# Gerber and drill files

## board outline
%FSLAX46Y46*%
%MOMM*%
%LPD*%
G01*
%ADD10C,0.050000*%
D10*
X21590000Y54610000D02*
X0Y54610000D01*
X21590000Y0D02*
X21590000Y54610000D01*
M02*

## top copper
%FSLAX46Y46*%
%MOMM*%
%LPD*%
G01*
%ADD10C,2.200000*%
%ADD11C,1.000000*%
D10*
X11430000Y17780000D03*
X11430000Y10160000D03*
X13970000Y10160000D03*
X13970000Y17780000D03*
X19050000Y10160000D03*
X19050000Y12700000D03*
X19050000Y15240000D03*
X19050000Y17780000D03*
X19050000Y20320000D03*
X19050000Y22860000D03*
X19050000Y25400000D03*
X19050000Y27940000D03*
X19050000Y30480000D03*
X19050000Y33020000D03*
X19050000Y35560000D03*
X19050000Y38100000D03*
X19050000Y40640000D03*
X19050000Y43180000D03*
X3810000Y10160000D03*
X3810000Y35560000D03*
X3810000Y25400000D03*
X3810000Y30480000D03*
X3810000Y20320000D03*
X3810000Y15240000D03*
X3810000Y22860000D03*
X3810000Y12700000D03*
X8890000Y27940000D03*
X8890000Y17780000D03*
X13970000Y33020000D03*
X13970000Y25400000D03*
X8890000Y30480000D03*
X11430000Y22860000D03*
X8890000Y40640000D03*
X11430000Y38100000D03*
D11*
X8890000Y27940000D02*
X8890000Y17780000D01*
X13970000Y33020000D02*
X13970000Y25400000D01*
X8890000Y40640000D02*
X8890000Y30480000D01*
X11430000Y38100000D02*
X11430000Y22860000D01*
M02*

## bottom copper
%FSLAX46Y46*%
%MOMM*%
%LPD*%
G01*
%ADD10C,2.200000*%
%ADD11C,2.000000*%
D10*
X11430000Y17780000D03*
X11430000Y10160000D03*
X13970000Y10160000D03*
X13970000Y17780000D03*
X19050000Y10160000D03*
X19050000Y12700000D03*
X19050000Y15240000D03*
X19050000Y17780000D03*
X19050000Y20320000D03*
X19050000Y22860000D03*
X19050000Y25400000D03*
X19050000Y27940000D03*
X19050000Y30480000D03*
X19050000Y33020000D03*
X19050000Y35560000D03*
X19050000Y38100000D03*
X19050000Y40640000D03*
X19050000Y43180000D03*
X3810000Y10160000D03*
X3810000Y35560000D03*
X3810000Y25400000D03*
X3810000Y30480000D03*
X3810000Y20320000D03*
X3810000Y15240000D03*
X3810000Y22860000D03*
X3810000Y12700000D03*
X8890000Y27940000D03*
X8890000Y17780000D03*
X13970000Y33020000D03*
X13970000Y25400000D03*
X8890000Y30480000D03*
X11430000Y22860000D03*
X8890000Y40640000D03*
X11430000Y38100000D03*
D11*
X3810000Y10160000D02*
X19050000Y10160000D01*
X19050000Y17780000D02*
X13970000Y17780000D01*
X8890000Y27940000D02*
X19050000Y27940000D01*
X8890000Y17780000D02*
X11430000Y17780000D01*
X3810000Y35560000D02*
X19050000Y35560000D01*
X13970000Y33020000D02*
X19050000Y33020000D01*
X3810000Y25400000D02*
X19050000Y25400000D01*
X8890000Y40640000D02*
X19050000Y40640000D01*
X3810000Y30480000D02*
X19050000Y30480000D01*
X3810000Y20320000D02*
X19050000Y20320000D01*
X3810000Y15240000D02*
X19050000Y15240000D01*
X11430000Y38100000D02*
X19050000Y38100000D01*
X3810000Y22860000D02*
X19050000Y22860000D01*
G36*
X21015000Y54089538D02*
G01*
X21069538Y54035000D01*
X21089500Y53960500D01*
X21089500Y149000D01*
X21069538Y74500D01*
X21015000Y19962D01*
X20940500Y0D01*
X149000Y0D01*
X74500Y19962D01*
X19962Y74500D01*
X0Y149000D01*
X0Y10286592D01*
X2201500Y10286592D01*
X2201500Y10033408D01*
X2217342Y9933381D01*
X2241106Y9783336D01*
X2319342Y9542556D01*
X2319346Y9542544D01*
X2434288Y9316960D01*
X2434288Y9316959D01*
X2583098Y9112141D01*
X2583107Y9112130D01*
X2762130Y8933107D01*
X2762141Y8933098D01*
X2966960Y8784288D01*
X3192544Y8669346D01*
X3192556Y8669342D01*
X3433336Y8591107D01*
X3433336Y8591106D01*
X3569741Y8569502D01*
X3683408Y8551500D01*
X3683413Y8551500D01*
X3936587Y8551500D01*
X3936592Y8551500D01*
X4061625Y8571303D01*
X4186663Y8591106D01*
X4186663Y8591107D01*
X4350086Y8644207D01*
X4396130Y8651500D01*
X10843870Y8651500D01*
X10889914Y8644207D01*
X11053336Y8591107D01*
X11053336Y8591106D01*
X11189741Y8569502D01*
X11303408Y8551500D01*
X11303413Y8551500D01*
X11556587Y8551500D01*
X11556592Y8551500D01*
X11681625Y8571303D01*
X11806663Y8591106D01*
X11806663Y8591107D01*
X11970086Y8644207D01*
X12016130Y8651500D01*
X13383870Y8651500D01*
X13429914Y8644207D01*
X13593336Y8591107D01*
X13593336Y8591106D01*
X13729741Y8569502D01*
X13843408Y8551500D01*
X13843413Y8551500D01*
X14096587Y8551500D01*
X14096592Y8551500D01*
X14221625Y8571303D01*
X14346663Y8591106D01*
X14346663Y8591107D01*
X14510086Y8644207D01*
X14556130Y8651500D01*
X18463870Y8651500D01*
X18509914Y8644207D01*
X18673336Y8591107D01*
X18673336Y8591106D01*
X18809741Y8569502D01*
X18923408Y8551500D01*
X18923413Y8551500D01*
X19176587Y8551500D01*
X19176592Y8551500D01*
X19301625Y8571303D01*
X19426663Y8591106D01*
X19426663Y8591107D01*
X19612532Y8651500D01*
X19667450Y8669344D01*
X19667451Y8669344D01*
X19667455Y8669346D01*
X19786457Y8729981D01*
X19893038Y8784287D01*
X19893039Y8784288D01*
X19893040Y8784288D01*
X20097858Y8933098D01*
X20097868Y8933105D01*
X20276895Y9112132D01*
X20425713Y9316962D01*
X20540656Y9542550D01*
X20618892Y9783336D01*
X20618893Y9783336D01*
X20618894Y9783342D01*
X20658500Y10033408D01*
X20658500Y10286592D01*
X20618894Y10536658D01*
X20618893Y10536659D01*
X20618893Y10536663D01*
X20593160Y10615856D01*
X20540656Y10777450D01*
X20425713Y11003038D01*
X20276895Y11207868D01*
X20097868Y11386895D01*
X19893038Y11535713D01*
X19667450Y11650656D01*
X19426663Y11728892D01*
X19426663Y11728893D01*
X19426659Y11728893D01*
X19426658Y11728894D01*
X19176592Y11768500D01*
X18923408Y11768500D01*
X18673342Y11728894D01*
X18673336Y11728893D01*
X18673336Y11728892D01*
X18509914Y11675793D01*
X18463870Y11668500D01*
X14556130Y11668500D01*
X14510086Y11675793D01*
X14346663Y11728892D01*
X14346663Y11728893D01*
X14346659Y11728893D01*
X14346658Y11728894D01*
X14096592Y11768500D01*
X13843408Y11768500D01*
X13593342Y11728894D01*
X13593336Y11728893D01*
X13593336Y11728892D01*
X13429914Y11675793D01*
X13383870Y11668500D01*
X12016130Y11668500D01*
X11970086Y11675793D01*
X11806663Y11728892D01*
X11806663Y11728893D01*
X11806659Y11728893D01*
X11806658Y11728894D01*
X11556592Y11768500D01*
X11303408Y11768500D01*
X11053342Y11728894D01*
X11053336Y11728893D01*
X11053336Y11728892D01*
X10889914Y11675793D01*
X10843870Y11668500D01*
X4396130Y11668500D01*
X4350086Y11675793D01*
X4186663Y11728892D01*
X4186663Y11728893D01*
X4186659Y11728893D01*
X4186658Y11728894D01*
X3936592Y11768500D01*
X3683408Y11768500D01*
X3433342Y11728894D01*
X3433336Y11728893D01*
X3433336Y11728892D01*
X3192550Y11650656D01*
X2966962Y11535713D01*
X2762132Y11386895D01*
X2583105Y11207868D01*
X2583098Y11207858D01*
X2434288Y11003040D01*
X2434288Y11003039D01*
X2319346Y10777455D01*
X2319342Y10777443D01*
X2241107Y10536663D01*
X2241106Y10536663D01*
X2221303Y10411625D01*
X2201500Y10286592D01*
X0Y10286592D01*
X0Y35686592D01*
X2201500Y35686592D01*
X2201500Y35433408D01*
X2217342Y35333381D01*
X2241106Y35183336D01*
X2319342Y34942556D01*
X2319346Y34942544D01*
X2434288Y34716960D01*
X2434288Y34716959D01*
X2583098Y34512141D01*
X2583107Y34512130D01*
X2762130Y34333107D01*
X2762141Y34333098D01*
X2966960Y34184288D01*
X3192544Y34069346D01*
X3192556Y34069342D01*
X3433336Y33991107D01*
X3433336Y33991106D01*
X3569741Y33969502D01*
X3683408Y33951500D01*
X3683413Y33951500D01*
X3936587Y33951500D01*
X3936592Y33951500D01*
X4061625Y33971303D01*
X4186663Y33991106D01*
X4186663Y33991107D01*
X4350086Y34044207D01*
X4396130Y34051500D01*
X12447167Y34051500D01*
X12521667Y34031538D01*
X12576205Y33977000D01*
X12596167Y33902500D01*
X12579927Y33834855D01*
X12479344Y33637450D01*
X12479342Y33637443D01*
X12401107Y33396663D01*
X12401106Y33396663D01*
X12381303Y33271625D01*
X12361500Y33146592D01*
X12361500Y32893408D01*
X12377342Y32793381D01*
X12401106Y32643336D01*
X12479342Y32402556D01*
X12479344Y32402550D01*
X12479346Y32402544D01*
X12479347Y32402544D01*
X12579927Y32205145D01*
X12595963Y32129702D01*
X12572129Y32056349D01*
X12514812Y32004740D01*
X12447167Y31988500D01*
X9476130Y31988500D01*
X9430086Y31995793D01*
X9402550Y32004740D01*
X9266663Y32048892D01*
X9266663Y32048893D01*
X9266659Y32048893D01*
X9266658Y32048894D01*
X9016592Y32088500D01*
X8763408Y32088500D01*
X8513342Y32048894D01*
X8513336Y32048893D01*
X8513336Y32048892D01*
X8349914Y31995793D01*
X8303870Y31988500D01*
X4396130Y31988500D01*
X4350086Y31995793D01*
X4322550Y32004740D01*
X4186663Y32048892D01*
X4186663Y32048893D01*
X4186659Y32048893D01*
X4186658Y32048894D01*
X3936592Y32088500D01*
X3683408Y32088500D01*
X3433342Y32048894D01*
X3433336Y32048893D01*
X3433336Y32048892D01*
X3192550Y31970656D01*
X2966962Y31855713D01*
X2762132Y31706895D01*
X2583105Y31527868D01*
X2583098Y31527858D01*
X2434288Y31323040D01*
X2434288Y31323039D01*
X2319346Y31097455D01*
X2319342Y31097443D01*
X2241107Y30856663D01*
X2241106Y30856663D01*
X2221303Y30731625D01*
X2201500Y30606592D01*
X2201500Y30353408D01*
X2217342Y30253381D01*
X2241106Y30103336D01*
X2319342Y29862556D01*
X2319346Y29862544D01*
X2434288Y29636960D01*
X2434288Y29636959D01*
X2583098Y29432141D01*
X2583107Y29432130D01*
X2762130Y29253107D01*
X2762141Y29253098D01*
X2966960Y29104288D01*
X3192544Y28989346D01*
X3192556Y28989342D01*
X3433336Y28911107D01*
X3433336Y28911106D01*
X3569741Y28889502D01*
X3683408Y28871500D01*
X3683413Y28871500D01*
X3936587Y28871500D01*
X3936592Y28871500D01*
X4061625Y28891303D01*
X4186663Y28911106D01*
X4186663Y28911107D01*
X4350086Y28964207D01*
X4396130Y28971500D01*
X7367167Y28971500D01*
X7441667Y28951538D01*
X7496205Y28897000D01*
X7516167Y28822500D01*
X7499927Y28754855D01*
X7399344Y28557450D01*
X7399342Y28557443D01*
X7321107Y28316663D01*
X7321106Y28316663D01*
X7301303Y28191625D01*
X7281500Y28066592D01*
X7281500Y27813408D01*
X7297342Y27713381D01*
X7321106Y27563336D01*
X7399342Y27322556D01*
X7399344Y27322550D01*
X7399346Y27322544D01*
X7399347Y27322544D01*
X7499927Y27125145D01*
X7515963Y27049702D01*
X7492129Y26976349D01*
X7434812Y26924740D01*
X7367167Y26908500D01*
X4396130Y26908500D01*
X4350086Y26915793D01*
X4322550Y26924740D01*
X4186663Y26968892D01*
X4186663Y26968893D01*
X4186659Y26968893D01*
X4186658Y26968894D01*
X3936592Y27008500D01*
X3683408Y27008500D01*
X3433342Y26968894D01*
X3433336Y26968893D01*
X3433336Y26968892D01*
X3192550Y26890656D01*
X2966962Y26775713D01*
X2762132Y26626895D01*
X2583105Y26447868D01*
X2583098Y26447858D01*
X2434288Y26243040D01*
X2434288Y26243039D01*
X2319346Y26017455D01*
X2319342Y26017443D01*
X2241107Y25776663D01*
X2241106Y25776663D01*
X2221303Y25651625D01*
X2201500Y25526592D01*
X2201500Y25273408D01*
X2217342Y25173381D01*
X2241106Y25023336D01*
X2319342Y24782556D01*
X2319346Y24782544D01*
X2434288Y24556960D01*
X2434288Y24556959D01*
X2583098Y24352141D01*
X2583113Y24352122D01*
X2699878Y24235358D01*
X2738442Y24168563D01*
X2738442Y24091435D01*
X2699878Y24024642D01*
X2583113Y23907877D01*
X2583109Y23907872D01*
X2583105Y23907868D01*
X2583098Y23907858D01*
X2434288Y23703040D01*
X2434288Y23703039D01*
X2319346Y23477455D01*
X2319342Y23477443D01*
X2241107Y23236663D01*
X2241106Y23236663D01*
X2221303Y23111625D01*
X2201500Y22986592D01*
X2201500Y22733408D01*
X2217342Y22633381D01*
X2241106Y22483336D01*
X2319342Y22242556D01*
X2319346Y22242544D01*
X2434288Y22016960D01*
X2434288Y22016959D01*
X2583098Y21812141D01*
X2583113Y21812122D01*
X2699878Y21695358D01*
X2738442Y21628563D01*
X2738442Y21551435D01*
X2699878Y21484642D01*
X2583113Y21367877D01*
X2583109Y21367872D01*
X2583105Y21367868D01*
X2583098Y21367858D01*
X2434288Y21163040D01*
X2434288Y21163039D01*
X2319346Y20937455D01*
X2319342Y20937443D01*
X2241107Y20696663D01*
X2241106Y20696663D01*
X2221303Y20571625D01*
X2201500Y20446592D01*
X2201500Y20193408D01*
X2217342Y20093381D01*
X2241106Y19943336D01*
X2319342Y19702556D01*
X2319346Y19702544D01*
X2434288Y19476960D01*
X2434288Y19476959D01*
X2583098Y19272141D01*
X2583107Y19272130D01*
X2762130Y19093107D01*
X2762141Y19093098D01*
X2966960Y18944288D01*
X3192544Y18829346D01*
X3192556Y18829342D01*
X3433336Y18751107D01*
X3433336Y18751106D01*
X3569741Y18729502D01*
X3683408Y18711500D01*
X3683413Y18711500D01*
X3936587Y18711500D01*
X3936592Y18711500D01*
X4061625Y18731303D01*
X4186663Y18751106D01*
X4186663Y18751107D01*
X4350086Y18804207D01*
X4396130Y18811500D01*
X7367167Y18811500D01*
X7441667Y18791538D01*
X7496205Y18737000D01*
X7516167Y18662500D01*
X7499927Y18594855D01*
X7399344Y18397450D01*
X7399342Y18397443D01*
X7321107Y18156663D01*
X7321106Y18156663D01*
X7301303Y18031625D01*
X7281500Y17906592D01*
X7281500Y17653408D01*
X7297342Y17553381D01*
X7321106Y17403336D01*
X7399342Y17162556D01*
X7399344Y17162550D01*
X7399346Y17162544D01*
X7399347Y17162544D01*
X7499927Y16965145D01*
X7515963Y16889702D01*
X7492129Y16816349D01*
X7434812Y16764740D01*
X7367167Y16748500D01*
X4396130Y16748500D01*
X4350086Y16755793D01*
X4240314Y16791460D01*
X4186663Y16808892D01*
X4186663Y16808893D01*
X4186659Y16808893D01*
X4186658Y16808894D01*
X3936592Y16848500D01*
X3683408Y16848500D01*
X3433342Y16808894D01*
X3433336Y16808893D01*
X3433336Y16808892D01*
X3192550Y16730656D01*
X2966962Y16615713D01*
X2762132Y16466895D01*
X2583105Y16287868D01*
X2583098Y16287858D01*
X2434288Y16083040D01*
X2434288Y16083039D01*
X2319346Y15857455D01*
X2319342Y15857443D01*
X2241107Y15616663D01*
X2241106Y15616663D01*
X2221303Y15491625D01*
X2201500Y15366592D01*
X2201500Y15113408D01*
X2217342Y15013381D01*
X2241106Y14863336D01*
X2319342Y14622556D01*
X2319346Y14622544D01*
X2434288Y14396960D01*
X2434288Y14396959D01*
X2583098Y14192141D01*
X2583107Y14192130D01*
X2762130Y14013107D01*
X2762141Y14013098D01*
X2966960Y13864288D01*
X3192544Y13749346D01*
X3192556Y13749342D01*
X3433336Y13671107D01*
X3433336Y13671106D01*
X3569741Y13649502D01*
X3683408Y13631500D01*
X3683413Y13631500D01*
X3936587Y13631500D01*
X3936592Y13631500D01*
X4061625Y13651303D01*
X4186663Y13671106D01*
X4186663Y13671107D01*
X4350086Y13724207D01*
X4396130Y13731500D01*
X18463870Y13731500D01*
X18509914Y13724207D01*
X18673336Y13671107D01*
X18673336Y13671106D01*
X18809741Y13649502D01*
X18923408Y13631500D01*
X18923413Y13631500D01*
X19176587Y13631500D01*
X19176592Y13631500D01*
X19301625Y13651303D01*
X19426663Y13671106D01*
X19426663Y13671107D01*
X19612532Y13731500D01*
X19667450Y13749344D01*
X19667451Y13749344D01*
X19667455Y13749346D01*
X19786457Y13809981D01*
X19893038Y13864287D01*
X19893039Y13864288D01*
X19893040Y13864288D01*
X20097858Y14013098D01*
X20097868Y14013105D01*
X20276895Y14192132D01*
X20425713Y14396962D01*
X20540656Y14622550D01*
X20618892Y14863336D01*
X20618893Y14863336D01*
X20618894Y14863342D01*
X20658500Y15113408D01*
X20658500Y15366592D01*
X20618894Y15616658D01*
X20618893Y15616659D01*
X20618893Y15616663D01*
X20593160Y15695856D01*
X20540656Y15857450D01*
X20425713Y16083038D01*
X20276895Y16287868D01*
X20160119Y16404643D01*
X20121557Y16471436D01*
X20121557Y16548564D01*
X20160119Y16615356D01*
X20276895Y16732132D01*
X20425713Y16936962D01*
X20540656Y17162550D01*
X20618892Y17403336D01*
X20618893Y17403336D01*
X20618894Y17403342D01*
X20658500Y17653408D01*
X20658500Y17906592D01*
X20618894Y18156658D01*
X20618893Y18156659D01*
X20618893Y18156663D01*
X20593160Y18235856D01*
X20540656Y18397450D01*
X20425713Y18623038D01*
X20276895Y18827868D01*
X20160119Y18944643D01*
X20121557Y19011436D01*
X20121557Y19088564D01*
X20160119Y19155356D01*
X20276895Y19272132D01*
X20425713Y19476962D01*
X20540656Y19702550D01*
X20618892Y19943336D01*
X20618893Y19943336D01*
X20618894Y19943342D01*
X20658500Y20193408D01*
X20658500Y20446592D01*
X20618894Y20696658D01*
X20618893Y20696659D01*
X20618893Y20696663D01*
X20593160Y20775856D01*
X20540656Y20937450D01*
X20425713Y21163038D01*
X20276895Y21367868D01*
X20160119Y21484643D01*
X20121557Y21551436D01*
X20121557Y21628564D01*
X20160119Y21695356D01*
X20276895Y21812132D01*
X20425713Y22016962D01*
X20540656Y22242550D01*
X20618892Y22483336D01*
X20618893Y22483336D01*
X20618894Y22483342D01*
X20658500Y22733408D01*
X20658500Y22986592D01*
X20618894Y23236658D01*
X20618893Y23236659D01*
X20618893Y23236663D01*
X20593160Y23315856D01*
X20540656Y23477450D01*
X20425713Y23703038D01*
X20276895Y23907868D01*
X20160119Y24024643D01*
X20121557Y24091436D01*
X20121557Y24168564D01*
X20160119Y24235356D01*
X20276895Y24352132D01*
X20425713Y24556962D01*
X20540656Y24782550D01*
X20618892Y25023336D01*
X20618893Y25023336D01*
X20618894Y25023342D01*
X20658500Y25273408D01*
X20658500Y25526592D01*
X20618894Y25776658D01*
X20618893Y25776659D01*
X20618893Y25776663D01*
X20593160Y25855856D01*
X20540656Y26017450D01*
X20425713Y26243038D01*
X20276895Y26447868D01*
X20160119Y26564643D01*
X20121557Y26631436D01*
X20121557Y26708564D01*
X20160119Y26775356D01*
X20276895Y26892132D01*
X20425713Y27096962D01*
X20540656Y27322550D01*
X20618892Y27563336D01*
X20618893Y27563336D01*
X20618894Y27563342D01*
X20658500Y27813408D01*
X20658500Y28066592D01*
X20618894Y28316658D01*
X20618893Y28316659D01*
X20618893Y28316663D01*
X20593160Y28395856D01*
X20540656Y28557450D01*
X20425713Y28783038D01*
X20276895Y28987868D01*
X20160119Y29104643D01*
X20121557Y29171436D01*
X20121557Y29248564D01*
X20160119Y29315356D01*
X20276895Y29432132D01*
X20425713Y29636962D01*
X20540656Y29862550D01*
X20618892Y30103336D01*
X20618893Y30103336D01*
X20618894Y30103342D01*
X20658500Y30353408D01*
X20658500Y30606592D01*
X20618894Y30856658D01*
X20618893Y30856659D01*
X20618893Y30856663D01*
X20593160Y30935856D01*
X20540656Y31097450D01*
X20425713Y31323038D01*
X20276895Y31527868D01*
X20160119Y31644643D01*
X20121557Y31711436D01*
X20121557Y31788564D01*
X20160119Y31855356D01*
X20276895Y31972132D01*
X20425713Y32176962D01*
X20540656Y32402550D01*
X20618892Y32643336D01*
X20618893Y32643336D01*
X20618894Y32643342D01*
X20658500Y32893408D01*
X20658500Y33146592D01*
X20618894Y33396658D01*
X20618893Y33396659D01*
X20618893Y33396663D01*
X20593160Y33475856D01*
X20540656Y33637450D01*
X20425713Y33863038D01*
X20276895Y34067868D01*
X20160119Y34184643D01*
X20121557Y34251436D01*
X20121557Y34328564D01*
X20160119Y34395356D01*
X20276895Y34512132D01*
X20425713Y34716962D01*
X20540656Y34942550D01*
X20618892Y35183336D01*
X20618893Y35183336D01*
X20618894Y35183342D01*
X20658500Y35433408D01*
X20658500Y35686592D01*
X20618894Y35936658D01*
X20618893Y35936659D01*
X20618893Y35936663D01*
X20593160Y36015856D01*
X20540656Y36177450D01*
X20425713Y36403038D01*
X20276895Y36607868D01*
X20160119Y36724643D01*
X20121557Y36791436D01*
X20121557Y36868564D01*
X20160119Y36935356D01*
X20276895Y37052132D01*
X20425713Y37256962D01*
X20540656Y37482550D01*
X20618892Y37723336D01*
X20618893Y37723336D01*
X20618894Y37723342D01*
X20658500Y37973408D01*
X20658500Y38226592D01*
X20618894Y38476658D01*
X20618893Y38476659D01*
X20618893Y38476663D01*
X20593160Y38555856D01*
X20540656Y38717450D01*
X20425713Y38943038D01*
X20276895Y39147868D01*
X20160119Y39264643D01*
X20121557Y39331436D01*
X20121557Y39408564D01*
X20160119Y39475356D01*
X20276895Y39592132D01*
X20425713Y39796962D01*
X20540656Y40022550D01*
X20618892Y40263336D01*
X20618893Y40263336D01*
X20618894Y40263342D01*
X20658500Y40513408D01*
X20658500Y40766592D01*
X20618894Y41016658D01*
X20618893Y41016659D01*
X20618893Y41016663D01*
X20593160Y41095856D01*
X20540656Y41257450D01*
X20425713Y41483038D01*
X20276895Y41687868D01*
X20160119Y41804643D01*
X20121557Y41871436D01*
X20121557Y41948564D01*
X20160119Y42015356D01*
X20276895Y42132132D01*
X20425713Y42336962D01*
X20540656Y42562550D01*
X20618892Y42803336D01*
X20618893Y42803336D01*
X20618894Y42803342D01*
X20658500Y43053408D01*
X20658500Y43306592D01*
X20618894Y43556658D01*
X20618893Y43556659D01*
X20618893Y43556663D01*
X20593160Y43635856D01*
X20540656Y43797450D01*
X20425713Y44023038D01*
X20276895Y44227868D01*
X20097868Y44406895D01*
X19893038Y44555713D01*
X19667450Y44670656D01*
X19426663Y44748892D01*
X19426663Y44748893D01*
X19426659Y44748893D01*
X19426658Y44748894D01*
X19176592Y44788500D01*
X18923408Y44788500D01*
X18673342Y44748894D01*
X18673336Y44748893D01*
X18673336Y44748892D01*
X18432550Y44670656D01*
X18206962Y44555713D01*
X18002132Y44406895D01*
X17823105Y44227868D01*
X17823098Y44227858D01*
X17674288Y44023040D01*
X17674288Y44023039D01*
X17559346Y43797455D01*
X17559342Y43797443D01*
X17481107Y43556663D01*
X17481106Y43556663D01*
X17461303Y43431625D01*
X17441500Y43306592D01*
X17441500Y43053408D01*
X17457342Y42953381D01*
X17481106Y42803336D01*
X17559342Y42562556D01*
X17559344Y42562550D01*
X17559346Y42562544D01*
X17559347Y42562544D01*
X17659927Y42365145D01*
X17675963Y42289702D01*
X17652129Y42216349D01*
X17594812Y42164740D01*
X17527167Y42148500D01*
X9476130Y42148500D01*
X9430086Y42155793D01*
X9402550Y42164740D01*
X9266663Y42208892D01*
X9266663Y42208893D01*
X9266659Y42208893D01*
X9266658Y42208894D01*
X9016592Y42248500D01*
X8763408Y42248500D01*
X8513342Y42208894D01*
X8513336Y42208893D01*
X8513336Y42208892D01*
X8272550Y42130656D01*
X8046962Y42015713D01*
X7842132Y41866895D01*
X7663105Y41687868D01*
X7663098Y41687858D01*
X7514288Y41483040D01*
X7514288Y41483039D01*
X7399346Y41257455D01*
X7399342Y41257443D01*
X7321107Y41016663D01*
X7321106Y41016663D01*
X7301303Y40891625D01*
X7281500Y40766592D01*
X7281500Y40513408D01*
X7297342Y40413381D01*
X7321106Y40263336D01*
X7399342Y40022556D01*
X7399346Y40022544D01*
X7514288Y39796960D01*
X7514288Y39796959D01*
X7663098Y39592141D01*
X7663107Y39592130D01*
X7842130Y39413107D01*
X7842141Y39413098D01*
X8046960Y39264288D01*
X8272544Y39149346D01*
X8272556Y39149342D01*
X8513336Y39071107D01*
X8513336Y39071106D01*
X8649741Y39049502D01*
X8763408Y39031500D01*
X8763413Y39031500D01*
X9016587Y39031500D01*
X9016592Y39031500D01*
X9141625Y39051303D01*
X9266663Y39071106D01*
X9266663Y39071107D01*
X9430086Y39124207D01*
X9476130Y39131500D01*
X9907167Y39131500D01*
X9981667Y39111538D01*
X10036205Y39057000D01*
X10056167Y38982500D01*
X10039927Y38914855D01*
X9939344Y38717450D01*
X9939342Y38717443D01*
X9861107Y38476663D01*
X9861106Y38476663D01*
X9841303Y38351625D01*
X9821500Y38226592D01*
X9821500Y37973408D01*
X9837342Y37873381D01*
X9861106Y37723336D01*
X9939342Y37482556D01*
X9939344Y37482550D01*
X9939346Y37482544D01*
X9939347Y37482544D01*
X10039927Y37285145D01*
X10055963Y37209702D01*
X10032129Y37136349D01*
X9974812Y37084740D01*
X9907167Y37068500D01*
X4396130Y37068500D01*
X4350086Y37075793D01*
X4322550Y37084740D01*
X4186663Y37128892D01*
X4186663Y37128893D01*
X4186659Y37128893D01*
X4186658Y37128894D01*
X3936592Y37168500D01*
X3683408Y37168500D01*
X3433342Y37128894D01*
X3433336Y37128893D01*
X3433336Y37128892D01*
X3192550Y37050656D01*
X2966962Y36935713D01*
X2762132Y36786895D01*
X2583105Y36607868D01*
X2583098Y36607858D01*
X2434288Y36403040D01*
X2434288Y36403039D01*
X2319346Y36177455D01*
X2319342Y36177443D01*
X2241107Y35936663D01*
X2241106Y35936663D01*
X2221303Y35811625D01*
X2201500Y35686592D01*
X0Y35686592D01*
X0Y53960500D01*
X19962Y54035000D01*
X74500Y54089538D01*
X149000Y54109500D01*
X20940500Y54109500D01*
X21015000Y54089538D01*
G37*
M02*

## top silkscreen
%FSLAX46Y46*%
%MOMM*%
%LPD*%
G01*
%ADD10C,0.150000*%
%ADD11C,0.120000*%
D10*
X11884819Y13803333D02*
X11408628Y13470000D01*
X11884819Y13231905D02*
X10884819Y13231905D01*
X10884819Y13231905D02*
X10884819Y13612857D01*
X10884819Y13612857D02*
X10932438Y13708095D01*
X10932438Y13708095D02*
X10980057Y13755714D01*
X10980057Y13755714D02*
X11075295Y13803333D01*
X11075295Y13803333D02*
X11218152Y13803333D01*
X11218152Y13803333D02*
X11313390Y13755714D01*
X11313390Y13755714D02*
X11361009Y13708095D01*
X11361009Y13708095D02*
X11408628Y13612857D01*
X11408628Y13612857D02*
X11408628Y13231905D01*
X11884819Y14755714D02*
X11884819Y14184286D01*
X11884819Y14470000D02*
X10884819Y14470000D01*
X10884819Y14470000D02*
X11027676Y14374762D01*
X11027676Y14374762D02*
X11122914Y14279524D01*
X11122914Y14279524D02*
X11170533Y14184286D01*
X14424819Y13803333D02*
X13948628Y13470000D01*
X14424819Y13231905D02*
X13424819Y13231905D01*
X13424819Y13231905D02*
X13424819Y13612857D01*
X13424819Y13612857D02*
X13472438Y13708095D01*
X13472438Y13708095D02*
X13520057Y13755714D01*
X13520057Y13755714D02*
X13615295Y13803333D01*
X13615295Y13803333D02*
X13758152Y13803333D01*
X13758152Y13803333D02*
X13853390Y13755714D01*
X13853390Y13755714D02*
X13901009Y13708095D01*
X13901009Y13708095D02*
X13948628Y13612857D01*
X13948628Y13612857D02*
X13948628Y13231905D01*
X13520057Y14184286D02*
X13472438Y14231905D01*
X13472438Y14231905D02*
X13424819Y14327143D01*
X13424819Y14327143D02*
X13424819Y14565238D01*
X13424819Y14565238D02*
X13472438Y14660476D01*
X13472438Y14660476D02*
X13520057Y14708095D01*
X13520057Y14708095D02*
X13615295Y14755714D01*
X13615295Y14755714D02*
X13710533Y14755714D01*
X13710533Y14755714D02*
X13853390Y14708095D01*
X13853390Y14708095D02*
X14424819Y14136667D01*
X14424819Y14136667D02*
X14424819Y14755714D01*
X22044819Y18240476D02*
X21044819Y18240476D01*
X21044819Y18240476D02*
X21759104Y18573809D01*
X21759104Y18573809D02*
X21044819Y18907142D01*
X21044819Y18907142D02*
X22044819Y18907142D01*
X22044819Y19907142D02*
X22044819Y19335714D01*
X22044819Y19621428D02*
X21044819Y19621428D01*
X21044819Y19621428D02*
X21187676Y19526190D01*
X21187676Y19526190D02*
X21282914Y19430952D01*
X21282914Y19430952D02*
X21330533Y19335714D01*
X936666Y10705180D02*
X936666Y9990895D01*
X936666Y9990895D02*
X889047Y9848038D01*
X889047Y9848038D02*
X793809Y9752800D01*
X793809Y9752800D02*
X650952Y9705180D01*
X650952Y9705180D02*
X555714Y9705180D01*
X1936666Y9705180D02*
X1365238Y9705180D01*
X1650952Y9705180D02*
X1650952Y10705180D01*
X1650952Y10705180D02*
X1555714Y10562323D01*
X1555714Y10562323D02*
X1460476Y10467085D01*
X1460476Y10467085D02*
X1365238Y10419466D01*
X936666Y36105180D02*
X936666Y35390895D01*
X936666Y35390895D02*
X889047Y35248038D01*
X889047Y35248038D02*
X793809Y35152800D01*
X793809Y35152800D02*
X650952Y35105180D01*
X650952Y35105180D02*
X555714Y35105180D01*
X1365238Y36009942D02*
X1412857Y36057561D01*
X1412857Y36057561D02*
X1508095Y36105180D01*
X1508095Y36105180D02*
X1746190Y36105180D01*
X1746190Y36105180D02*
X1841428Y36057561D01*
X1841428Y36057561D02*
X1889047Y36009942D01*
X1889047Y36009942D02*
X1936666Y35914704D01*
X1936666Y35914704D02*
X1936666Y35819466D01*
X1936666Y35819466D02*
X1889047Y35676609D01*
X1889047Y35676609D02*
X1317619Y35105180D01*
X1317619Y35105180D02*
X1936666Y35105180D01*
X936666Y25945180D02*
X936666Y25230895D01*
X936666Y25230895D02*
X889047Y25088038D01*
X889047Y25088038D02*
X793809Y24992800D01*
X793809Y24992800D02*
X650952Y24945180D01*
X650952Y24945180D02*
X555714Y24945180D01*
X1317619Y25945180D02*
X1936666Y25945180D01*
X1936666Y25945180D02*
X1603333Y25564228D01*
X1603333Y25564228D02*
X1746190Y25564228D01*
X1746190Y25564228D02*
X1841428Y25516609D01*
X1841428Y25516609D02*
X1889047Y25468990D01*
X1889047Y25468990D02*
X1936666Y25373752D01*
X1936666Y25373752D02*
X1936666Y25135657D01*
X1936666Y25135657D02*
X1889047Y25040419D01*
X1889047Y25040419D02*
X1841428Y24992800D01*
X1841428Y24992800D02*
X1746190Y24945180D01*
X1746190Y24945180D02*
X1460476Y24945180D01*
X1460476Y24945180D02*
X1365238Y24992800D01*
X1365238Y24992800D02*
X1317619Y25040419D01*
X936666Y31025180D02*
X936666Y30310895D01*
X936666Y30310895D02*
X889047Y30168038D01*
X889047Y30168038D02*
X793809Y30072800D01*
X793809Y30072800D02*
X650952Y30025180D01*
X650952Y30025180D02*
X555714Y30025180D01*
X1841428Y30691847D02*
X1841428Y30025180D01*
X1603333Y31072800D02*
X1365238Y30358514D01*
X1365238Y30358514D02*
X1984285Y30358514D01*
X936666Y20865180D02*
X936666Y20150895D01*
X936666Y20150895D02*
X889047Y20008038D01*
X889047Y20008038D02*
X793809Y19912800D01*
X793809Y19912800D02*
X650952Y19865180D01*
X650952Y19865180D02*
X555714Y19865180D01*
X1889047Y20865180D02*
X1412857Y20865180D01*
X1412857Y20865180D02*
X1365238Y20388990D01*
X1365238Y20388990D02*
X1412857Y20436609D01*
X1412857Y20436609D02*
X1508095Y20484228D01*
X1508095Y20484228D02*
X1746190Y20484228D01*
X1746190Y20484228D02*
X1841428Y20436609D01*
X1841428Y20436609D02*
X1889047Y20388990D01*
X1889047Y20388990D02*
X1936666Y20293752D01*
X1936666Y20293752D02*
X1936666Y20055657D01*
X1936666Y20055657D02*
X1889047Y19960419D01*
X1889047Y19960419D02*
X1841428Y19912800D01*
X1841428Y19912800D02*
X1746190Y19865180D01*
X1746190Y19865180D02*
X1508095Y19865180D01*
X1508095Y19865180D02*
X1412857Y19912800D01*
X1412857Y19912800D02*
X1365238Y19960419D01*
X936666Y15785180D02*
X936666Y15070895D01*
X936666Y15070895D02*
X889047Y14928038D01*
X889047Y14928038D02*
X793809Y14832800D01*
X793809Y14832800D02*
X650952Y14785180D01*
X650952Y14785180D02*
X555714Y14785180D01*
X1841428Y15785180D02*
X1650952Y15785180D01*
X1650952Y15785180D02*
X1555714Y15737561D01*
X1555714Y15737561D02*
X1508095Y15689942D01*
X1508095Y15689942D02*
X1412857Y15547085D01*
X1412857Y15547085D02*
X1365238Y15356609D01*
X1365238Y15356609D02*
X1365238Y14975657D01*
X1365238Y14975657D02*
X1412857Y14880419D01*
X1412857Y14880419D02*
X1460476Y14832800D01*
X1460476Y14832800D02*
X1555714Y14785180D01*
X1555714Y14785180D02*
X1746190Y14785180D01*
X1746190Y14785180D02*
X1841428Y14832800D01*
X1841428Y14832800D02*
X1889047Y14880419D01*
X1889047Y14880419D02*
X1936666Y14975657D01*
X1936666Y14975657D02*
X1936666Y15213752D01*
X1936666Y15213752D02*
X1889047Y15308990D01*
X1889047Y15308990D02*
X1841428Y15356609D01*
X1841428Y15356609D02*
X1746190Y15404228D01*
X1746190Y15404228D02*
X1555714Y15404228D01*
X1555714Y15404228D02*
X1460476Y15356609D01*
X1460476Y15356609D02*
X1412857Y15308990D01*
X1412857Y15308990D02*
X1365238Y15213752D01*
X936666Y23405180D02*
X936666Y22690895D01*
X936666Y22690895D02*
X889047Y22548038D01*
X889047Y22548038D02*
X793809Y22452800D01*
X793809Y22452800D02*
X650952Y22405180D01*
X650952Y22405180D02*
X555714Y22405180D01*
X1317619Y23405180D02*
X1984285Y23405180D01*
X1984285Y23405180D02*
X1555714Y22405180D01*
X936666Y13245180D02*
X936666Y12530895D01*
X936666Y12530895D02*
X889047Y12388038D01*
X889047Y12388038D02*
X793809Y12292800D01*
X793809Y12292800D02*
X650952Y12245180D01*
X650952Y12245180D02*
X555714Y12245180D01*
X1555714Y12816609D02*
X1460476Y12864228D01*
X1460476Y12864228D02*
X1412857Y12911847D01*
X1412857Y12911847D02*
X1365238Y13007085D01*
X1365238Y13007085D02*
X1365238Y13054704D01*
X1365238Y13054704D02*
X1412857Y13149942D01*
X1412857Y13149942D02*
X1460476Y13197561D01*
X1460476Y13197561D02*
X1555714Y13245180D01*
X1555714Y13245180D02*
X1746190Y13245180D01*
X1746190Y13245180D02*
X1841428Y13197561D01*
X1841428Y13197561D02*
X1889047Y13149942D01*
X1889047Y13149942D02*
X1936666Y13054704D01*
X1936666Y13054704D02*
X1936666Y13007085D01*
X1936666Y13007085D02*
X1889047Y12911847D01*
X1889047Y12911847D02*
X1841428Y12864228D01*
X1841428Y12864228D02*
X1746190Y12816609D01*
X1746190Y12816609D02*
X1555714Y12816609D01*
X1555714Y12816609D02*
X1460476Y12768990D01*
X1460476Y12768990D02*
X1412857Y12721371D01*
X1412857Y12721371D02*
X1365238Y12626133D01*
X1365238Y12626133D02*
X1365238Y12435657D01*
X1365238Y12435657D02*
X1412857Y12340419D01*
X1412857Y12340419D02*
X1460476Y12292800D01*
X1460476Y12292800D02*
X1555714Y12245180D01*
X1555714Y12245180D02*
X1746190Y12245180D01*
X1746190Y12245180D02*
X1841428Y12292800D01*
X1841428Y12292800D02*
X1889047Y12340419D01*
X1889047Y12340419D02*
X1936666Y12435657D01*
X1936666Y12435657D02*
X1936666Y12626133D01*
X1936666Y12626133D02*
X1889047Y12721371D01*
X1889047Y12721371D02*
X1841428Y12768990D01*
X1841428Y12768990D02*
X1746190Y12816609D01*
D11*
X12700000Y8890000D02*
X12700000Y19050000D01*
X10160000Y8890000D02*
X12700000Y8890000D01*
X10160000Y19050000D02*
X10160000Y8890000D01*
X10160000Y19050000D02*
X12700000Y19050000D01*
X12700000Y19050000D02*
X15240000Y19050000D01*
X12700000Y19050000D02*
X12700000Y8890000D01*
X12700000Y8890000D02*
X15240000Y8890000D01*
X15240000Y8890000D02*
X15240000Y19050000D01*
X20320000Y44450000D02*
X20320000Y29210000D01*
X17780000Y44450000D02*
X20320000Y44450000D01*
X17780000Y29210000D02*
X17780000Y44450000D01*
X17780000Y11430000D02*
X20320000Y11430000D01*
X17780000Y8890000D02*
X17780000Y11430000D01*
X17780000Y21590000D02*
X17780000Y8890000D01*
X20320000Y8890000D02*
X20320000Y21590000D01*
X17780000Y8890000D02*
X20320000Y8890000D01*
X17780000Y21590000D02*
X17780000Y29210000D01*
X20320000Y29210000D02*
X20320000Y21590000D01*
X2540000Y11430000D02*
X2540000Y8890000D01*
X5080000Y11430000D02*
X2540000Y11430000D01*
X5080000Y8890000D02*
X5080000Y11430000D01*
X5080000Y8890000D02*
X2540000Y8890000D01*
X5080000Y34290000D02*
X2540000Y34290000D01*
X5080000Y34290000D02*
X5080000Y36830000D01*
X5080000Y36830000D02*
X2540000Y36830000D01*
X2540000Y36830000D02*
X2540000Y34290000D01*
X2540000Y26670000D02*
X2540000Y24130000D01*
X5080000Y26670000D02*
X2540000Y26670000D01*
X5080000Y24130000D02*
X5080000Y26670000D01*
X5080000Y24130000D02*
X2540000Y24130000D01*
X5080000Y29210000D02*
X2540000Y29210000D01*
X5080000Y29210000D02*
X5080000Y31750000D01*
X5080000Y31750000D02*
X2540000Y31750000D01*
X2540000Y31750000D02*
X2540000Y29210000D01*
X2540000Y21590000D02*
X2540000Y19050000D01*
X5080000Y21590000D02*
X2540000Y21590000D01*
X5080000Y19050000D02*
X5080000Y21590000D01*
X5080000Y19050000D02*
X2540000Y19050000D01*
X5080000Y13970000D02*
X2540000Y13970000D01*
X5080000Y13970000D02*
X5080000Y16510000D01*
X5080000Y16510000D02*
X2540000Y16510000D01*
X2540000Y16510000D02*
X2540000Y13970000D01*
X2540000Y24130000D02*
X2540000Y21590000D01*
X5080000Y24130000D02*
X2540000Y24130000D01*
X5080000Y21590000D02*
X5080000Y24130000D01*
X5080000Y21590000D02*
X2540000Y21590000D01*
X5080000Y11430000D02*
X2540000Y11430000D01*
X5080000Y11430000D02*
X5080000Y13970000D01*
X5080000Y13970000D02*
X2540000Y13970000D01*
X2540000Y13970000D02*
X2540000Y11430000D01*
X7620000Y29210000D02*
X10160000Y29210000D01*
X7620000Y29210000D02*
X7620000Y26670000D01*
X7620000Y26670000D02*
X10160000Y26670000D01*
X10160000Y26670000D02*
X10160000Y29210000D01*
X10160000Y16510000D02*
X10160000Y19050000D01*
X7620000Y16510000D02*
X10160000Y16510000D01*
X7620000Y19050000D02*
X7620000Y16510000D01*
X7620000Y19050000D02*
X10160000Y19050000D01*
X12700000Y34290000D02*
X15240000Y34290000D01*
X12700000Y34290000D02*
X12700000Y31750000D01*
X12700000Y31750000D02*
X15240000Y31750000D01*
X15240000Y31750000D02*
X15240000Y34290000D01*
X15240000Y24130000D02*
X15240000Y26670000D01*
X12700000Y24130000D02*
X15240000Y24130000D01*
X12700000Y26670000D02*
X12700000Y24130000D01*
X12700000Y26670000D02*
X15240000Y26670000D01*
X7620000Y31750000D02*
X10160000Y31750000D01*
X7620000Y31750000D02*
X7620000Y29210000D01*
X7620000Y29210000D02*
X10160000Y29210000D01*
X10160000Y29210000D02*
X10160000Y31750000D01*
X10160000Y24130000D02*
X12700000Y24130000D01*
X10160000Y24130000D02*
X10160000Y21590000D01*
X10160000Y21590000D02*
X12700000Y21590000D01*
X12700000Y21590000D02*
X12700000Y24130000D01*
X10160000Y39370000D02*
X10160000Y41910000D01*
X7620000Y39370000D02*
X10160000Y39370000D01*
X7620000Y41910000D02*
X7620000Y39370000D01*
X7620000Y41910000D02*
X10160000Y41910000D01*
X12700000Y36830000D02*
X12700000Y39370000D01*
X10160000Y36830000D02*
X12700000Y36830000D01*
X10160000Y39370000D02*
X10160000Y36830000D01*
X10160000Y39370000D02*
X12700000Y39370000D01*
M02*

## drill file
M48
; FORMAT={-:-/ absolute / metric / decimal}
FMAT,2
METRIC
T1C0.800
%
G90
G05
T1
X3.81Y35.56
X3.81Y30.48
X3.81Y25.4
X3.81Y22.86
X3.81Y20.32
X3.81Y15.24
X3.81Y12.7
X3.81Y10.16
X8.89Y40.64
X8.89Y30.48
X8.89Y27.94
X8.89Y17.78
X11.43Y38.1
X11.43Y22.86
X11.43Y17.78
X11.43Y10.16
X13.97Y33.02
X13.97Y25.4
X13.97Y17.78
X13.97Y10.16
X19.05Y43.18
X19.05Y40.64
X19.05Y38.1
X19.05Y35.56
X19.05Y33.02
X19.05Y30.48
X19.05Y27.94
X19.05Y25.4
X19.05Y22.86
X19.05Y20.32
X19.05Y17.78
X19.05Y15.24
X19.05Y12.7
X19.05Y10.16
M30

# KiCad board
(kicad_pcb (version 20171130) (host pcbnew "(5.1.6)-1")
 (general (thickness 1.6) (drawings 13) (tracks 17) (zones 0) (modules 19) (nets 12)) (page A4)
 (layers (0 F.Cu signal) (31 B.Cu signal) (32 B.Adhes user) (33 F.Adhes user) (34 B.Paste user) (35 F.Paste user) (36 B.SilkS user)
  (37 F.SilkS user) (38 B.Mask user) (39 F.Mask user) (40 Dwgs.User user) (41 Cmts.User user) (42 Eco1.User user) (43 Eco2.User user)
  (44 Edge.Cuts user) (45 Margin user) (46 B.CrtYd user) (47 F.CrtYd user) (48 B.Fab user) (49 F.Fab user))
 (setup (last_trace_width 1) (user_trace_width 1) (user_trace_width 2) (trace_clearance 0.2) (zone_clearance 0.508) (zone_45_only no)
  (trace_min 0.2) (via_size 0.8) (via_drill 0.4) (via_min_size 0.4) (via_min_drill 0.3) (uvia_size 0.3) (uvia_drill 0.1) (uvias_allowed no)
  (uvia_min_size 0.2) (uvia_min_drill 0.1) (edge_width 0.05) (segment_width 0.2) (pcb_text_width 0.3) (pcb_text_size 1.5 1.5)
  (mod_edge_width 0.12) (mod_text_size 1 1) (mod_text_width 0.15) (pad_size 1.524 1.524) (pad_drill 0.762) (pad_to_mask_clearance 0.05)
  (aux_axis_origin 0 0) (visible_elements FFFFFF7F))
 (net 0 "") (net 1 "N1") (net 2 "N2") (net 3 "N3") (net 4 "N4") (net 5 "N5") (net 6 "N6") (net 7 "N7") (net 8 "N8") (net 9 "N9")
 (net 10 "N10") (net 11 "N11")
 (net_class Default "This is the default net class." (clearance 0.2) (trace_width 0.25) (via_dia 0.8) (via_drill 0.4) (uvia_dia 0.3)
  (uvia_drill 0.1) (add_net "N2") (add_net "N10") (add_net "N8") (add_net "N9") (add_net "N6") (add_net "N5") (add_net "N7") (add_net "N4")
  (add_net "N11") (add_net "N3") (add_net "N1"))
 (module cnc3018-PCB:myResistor (layer F.Cu) (at 11.43 -10.16 90)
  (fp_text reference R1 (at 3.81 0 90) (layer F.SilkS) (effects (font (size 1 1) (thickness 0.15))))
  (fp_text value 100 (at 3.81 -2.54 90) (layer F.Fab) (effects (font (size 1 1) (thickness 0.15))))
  (fp_line (start -1.27 1.27) (end 8.89 1.27) (layer F.SilkS) (width 0.12))
  (fp_line (start -1.27 -1.27) (end -1.27 1.27) (layer F.SilkS) (width 0.12))
  (fp_line (start 8.89 -1.27) (end -1.27 -1.27) (layer F.SilkS) (width 0.12))
  (fp_line (start 8.89 -1.27) (end 8.89 1.27) (layer F.SilkS) (width 0.12))
  (pad 2 thru_hole circle (at 7.62 0 90) (size 2.2 2.2) (drill 0.8) (layers *.Cu *.Mask) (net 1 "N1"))
  (pad 1 thru_hole circle (at 0 0 90) (size 2.2 2.2) (drill 0.8) (layers *.Cu *.Mask) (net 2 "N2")))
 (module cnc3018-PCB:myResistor (layer F.Cu) (at 13.97 -10.16 90)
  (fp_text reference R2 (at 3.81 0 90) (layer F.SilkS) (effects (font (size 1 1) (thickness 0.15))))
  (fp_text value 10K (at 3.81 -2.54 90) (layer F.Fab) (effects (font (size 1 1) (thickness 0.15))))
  (fp_line (start 8.89 -1.27) (end 8.89 1.27) (layer F.SilkS) (width 0.12))
  (fp_line (start 8.89 -1.27) (end -1.27 -1.27) (layer F.SilkS) (width 0.12))
  (fp_line (start -1.27 -1.27) (end -1.27 1.27) (layer F.SilkS) (width 0.12))
  (fp_line (start -1.27 1.27) (end 8.89 1.27) (layer F.SilkS) (width 0.12))
  (pad 1 thru_hole circle (at 0 0 90) (size 2.2 2.2) (drill 0.8) (layers *.Cu *.Mask) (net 2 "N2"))
  (pad 2 thru_hole circle (at 7.62 0 90) (size 2.2 2.2) (drill 0.8) (layers *.Cu *.Mask) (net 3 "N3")))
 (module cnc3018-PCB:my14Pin (layer F.Cu) (at 19.05 -17.78 90)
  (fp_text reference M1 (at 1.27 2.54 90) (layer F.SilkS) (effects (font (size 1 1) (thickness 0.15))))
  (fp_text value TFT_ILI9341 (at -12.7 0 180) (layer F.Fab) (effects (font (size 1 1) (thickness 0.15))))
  (fp_line (start 26.67 1.27) (end 11.43 1.27) (layer F.SilkS) (width 0.12))
  (fp_line (start 26.67 -1.27) (end 26.67 1.27) (layer F.SilkS) (width 0.12))
  (fp_line (start 11.43 -1.27) (end 26.67 -1.27) (layer F.SilkS) (width 0.12))
  (fp_line (start -6.35 -1.27) (end -6.35 1.27) (layer F.SilkS) (width 0.12))
  (fp_line (start -8.89 -1.27) (end -6.35 -1.27) (layer F.SilkS) (width 0.12))
  (fp_line (start 3.81 -1.27) (end -8.89 -1.27) (layer F.SilkS) (width 0.12))
  (fp_line (start -8.89 1.27) (end 3.81 1.27) (layer F.SilkS) (width 0.12))
  (fp_line (start -8.89 -1.27) (end -8.89 1.27) (layer F.SilkS) (width 0.12))
  (fp_line (start 3.81 -1.27) (end 11.43 -1.27) (layer F.SilkS) (width 0.12))
  (fp_line (start 11.43 1.27) (end 3.81 1.27) (layer F.SilkS) (width 0.12))
  (pad 1 thru_hole circle (at -7.62 0 90) (size 2.2 2.2) (drill 0.8) (layers *.Cu *.Mask) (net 2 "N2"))
  (pad 2 thru_hole circle (at -5.08 0 90) (size 2.2 2.2) (drill 0.8) (layers *.Cu *.Mask) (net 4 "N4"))
  (pad 3 thru_hole circle (at -2.54 0 90) (size 2.2 2.2) (drill 0.8) (layers *.Cu *.Mask) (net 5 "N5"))
  (pad 4 thru_hole circle (at 0 0 90) (size 2.2 2.2) (drill 0.8) (layers *.Cu *.Mask) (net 3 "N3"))
  (pad 5 thru_hole circle (at 2.54 0 90) (size 2.2 2.2) (drill 0.8) (layers *.Cu *.Mask) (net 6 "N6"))
  (pad 6 thru_hole circle (at 5.08 0 90) (size 2.2 2.2) (drill 0.8) (layers *.Cu *.Mask) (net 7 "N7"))
  (pad 7 thru_hole circle (at 7.62 0 90) (size 2.2 2.2) (drill 0.8) (layers *.Cu *.Mask) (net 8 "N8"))
  (pad 8 thru_hole circle (at 10.16 0 90) (size 2.2 2.2) (drill 0.8) (layers *.Cu *.Mask) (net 1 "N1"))
  (pad 9 thru_hole circle (at 12.7 0 90) (size 2.2 2.2) (drill 0.8) (layers *.Cu *.Mask) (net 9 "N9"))
  (pad 10 thru_hole circle (at 15.24 0 90) (size 2.2 2.2) (drill 0.8) (layers *.Cu *.Mask) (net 8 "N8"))
  (pad 11 thru_hole circle (at 17.78 0 90) (size 2.2 2.2) (drill 0.8) (layers *.Cu *.Mask) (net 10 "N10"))
  (pad 12 thru_hole circle (at 20.32 0 90) (size 2.2 2.2) (drill 0.8) (layers *.Cu *.Mask) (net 7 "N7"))
  (pad 13 thru_hole circle (at 22.86 0 90) (size 2.2 2.2) (drill 0.8) (layers *.Cu *.Mask) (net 9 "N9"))
  (pad 14 thru_hole circle (at 25.4 0 90) (size 2.2 2.2) (drill 0.8) (layers *.Cu *.Mask) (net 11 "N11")))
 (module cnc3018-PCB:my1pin (layer F.Cu) (at 3.81 -10.16 180)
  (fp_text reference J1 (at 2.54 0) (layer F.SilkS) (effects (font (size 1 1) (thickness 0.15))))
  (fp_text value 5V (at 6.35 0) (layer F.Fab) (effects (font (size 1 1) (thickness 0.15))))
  (fp_line (start 1.27 1.27) (end 1.27 -1.27) (layer F.SilkS) (width 0.12))
  (fp_line (start -1.27 1.27) (end 1.27 1.27) (layer F.SilkS) (width 0.12))
  (fp_line (start -1.27 -1.27) (end -1.27 1.27) (layer F.SilkS) (width 0.12))
  (fp_line (start -1.27 -1.27) (end 1.27 -1.27) (layer F.SilkS) (width 0.12))
  (pad 1 thru_hole circle (at 0 0 180) (size 2.2 2.2) (drill 0.8) (layers *.Cu *.Mask) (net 2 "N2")))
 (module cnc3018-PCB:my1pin (layer F.Cu) (at 3.81 -35.56 180)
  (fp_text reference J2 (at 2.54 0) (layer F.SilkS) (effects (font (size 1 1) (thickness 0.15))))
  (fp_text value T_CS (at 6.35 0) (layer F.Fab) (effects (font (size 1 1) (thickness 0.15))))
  (fp_line (start -1.27 -1.27) (end 1.27 -1.27) (layer F.SilkS) (width 0.12))
  (fp_line (start -1.27 -1.27) (end -1.27 1.27) (layer F.SilkS) (width 0.12))
  (fp_line (start -1.27 1.27) (end 1.27 1.27) (layer F.SilkS) (width 0.12))
  (fp_line (start 1.27 1.27) (end 1.27 -1.27) (layer F.SilkS) (width 0.12))
  (pad 1 thru_hole circle (at 0 0 180) (size 2.2 2.2) (drill 0.8) (layers *.Cu *.Mask) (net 10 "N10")))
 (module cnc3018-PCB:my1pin (layer F.Cu) (at 3.81 -25.4 180)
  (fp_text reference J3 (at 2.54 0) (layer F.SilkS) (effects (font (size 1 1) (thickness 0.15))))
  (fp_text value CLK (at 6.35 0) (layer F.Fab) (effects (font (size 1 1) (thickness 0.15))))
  (fp_line (start 1.27 1.27) (end 1.27 -1.27) (layer F.SilkS) (width 0.12))
  (fp_line (start -1.27 1.27) (end 1.27 1.27) (layer F.SilkS) (width 0.12))
  (fp_line (start -1.27 -1.27) (end -1.27 1.27) (layer F.SilkS) (width 0.12))
  (fp_line (start -1.27 -1.27) (end 1.27 -1.27) (layer F.SilkS) (width 0.12))
  (pad 1 thru_hole circle (at 0 0 180) (size 2.2 2.2) (drill 0.8) (layers *.Cu *.Mask) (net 8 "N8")))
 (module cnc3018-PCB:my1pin (layer F.Cu) (at 3.81 -30.48 180)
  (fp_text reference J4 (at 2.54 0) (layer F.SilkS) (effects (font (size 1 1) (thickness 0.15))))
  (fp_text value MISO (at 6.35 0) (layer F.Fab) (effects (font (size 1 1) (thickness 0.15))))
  (fp_line (start -1.27 -1.27) (end 1.27 -1.27) (layer F.SilkS) (width 0.12))
  (fp_line (start -1.27 -1.27) (end -1.27 1.27) (layer F.SilkS) (width 0.12))
  (fp_line (start -1.27 1.27) (end 1.27 1.27) (layer F.SilkS) (width 0.12))
  (fp_line (start 1.27 1.27) (end 1.27 -1.27) (layer F.SilkS) (width 0.12))
  (pad 1 thru_hole circle (at 0 0 180) (size 2.2 2.2) (drill 0.8) (layers *.Cu *.Mask) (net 9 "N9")))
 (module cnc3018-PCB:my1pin (layer F.Cu) (at 3.81 -20.32 180)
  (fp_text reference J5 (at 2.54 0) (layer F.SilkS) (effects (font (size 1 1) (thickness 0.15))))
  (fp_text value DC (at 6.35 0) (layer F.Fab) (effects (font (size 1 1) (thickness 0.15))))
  (fp_line (start 1.27 1.27) (end 1.27 -1.27) (layer F.SilkS) (width 0.12))
  (fp_line (start -1.27 1.27) (end 1.27 1.27) (layer F.SilkS) (width 0.12))
  (fp_line (start -1.27 -1.27) (end -1.27 1.27) (layer F.SilkS) (width 0.12))
  (fp_line (start -1.27 -1.27) (end 1.27 -1.27) (layer F.SilkS) (width 0.12))
  (pad 1 thru_hole circle (at 0 0 180) (size 2.2 2.2) (drill 0.8) (layers *.Cu *.Mask) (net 6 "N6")))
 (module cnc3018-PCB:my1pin (layer F.Cu) (at 3.81 -15.24 180)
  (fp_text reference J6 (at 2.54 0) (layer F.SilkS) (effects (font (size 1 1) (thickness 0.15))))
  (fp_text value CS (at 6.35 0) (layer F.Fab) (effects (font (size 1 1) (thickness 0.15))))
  (fp_line (start -1.27 -1.27) (end 1.27 -1.27) (layer F.SilkS) (width 0.12))
  (fp_line (start -1.27 -1.27) (end -1.27 1.27) (layer F.SilkS) (width 0.12))
  (fp_line (start -1.27 1.27) (end 1.27 1.27) (layer F.SilkS) (width 0.12))
  (fp_line (start 1.27 1.27) (end 1.27 -1.27) (layer F.SilkS) (width 0.12))
  (pad 1 thru_hole circle (at 0 0 180) (size 2.2 2.2) (drill 0.8) (layers *.Cu *.Mask) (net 5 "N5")))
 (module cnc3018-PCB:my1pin (layer F.Cu) (at 3.81 -22.86 180)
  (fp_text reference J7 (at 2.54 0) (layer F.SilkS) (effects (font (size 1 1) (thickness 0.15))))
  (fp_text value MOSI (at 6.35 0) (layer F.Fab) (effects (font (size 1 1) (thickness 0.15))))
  (fp_line (start 1.27 1.27) (end 1.27 -1.27) (layer F.SilkS) (width 0.12))
  (fp_line (start -1.27 1.27) (end 1.27 1.27) (layer F.SilkS) (width 0.12))
  (fp_line (start -1.27 -1.27) (end -1.27 1.27) (layer F.SilkS) (width 0.12))
  (fp_line (start -1.27 -1.27) (end 1.27 -1.27) (layer F.SilkS) (width 0.12))
  (pad 1 thru_hole circle (at 0 0 180) (size 2.2 2.2) (drill 0.8) (layers *.Cu *.Mask) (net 7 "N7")))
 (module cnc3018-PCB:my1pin (layer F.Cu) (at 3.81 -12.7 180)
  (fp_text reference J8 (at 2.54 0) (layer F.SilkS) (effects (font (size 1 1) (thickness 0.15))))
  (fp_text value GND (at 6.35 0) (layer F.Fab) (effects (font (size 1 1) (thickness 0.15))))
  (fp_line (start -1.27 -1.27) (end 1.27 -1.27) (layer F.SilkS) (width 0.12))
  (fp_line (start -1.27 -1.27) (end -1.27 1.27) (layer F.SilkS) (width 0.12))
  (fp_line (start -1.27 1.27) (end 1.27 1.27) (layer F.SilkS) (width 0.12))
  (fp_line (start 1.27 1.27) (end 1.27 -1.27) (layer F.SilkS) (width 0.12))
  (pad 1 thru_hole circle (at 0 0 180) (size 2.2 2.2) (drill 0.8) (layers *.Cu *.Mask) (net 4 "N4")))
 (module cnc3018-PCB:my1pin (layer F.Cu) (at 8.89 -27.94)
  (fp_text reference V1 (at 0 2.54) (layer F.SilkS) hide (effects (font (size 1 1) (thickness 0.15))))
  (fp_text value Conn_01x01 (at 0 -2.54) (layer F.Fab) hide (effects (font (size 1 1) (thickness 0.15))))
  (fp_line (start -1.27 -1.27) (end 1.27 -1.27) (layer F.SilkS) (width 0.12))
  (fp_line (start -1.27 -1.27) (end -1.27 1.27) (layer F.SilkS) (width 0.12))
  (fp_line (start -1.27 1.27) (end 1.27 1.27) (layer F.SilkS) (width 0.12))
  (fp_line (start 1.27 1.27) (end 1.27 -1.27) (layer F.SilkS) (width 0.12))
  (pad 1 thru_hole circle (at 0 0) (size 2.2 2.2) (drill 0.8) (layers *.Cu *.Mask) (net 1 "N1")))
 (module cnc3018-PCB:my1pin (layer F.Cu) (at 8.89 -17.78)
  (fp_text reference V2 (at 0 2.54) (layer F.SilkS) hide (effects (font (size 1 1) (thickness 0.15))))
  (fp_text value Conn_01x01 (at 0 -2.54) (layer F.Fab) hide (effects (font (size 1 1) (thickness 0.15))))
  (fp_line (start 1.27 1.27) (end 1.27 -1.27) (layer F.SilkS) (width 0.12))
  (fp_line (start -1.27 1.27) (end 1.27 1.27) (layer F.SilkS) (width 0.12))
  (fp_line (start -1.27 -1.27) (end -1.27 1.27) (layer F.SilkS) (width 0.12))
  (fp_line (start -1.27 -1.27) (end 1.27 -1.27) (layer F.SilkS) (width 0.12))
  (pad 1 thru_hole circle (at 0 0) (size 2.2 2.2) (drill 0.8) (layers *.Cu *.Mask) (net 1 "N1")))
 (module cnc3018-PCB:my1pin (layer F.Cu) (at 13.97 -33.02)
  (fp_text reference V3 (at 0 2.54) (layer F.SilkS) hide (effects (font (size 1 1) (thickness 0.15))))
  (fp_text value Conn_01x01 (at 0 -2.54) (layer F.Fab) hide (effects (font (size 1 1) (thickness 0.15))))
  (fp_line (start -1.27 -1.27) (end 1.27 -1.27) (layer F.SilkS) (width 0.12))
  (fp_line (start -1.27 -1.27) (end -1.27 1.27) (layer F.SilkS) (width 0.12))
  (fp_line (start -1.27 1.27) (end 1.27 1.27) (layer F.SilkS) (width 0.12))
  (fp_line (start 1.27 1.27) (end 1.27 -1.27) (layer F.SilkS) (width 0.12))
  (pad 1 thru_hole circle (at 0 0) (size 2.2 2.2) (drill 0.8) (layers *.Cu *.Mask) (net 8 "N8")))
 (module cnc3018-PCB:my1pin (layer F.Cu) (at 13.97 -25.4)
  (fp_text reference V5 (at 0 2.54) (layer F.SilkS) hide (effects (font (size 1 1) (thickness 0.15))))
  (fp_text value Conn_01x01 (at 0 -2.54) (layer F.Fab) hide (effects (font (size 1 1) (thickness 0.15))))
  (fp_line (start 1.27 1.27) (end 1.27 -1.27) (layer F.SilkS) (width 0.12))
  (fp_line (start -1.27 1.27) (end 1.27 1.27) (layer F.SilkS) (width 0.12))
  (fp_line (start -1.27 -1.27) (end -1.27 1.27) (layer F.SilkS) (width 0.12))
  (fp_line (start -1.27 -1.27) (end 1.27 -1.27) (layer F.SilkS) (width 0.12))
  (pad 1 thru_hole circle (at 0 0) (size 2.2 2.2) (drill 0.8) (layers *.Cu *.Mask) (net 8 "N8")))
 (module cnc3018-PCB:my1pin (layer F.Cu) (at 8.89 -30.48)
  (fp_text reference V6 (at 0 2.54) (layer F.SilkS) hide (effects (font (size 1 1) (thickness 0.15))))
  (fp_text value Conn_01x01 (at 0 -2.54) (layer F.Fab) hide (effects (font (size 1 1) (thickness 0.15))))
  (fp_line (start -1.27 -1.27) (end 1.27 -1.27) (layer F.SilkS) (width 0.12))
  (fp_line (start -1.27 -1.27) (end -1.27 1.27) (layer F.SilkS) (width 0.12))
  (fp_line (start -1.27 1.27) (end 1.27 1.27) (layer F.SilkS) (width 0.12))
  (fp_line (start 1.27 1.27) (end 1.27 -1.27) (layer F.SilkS) (width 0.12))
  (pad 1 thru_hole circle (at 0 0) (size 2.2 2.2) (drill 0.8) (layers *.Cu *.Mask) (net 9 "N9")))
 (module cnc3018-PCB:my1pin (layer F.Cu) (at 11.43 -22.86)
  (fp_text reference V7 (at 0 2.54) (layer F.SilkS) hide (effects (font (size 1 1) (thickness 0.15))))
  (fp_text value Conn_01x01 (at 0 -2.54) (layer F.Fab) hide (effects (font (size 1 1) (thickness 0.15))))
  (fp_line (start -1.27 -1.27) (end 1.27 -1.27) (layer F.SilkS) (width 0.12))
  (fp_line (start -1.27 -1.27) (end -1.27 1.27) (layer F.SilkS) (width 0.12))
  (fp_line (start -1.27 1.27) (end 1.27 1.27) (layer F.SilkS) (width 0.12))
  (fp_line (start 1.27 1.27) (end 1.27 -1.27) (layer F.SilkS) (width 0.12))
  (pad 1 thru_hole circle (at 0 0) (size 2.2 2.2) (drill 0.8) (layers *.Cu *.Mask) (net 7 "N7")))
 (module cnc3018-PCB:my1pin (layer F.Cu) (at 8.89 -40.64)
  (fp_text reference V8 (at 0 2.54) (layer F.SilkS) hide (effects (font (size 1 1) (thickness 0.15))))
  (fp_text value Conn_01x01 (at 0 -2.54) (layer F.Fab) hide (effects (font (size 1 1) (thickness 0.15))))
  (fp_line (start 1.27 1.27) (end 1.27 -1.27) (layer F.SilkS) (width 0.12))
  (fp_line (start -1.27 1.27) (end 1.27 1.27) (layer F.SilkS) (width 0.12))
  (fp_line (start -1.27 -1.27) (end -1.27 1.27) (layer F.SilkS) (width 0.12))
  (fp_line (start -1.27 -1.27) (end 1.27 -1.27) (layer F.SilkS) (width 0.12))
  (pad 1 thru_hole circle (at 0 0) (size 2.2 2.2) (drill 0.8) (layers *.Cu *.Mask) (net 9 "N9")))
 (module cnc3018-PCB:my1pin (layer F.Cu) (at 11.43 -38.1)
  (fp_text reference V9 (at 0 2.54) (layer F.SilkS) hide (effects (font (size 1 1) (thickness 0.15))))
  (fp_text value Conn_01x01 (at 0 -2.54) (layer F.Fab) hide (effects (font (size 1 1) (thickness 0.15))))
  (fp_line (start 1.27 1.27) (end 1.27 -1.27) (layer F.SilkS) (width 0.12))
  (fp_line (start -1.27 1.27) (end 1.27 1.27) (layer F.SilkS) (width 0.12))
  (fp_line (start -1.27 -1.27) (end -1.27 1.27) (layer F.SilkS) (width 0.12))
  (fp_line (start -1.27 -1.27) (end 1.27 -1.27) (layer F.SilkS) (width 0.12))
  (pad 1 thru_hole circle (at 0 0) (size 2.2 2.2) (drill 0.8) (layers *.Cu *.Mask) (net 7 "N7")))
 (gr_line (start 21.59 -54.61) (end 0 -54.61) (layer Edge.Cuts) (width 0.05))
 (gr_line (start 21.59 0) (end 21.59 -54.61) (layer Edge.Cuts) (width 0.05))
 (segment (start 3.81 -10.16) (end 19.05 -10.16) (width 2) (layer B.Cu) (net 2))
 (segment (start 19.05 -17.78) (end 13.97 -17.78) (width 2) (layer B.Cu) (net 3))
 (segment (start 8.89 -27.94) (end 19.05 -27.94) (width 2) (layer B.Cu) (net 1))
 (segment (start 8.89 -17.78) (end 11.43 -17.78) (width 2) (layer B.Cu) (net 1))
 (segment (start 8.89 -27.94) (end 8.89 -17.78) (width 1) (layer F.Cu) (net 1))
 (segment (start 3.81 -35.56) (end 19.05 -35.56) (width 2) (layer B.Cu) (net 10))
 (segment (start 13.97 -33.02) (end 19.05 -33.02) (width 2) (layer B.Cu) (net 8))
 (segment (start 3.81 -25.4) (end 19.05 -25.4) (width 2) (layer B.Cu) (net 8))
 (segment (start 13.97 -33.02) (end 13.97 -25.4) (width 1) (layer F.Cu) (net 8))
 (segment (start 8.89 -40.64) (end 19.05 -40.64) (width 2) (layer B.Cu) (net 9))
 (segment (start 3.81 -30.48) (end 19.05 -30.48) (width 2) (layer B.Cu) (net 9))
 (segment (start 8.89 -40.64) (end 8.89 -30.48) (width 1) (layer F.Cu) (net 9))
 (segment (start 3.81 -20.32) (end 19.05 -20.32) (width 2) (layer B.Cu) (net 6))
 (segment (start 3.81 -15.24) (end 19.05 -15.24) (width 2) (layer B.Cu) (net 5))
 (segment (start 11.43 -38.1) (end 19.05 -38.1) (width 2) (layer B.Cu) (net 7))
 (segment (start 3.81 -22.86) (end 19.05 -22.86) (width 2) (layer B.Cu) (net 7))
 (segment (start 11.43 -38.1) (end 11.43 -22.86) (width 1) (layer F.Cu) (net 7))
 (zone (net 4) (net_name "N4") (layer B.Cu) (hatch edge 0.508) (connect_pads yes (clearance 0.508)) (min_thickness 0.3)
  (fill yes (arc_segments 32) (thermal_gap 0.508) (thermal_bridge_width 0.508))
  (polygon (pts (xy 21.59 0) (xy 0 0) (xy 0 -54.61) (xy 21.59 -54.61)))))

